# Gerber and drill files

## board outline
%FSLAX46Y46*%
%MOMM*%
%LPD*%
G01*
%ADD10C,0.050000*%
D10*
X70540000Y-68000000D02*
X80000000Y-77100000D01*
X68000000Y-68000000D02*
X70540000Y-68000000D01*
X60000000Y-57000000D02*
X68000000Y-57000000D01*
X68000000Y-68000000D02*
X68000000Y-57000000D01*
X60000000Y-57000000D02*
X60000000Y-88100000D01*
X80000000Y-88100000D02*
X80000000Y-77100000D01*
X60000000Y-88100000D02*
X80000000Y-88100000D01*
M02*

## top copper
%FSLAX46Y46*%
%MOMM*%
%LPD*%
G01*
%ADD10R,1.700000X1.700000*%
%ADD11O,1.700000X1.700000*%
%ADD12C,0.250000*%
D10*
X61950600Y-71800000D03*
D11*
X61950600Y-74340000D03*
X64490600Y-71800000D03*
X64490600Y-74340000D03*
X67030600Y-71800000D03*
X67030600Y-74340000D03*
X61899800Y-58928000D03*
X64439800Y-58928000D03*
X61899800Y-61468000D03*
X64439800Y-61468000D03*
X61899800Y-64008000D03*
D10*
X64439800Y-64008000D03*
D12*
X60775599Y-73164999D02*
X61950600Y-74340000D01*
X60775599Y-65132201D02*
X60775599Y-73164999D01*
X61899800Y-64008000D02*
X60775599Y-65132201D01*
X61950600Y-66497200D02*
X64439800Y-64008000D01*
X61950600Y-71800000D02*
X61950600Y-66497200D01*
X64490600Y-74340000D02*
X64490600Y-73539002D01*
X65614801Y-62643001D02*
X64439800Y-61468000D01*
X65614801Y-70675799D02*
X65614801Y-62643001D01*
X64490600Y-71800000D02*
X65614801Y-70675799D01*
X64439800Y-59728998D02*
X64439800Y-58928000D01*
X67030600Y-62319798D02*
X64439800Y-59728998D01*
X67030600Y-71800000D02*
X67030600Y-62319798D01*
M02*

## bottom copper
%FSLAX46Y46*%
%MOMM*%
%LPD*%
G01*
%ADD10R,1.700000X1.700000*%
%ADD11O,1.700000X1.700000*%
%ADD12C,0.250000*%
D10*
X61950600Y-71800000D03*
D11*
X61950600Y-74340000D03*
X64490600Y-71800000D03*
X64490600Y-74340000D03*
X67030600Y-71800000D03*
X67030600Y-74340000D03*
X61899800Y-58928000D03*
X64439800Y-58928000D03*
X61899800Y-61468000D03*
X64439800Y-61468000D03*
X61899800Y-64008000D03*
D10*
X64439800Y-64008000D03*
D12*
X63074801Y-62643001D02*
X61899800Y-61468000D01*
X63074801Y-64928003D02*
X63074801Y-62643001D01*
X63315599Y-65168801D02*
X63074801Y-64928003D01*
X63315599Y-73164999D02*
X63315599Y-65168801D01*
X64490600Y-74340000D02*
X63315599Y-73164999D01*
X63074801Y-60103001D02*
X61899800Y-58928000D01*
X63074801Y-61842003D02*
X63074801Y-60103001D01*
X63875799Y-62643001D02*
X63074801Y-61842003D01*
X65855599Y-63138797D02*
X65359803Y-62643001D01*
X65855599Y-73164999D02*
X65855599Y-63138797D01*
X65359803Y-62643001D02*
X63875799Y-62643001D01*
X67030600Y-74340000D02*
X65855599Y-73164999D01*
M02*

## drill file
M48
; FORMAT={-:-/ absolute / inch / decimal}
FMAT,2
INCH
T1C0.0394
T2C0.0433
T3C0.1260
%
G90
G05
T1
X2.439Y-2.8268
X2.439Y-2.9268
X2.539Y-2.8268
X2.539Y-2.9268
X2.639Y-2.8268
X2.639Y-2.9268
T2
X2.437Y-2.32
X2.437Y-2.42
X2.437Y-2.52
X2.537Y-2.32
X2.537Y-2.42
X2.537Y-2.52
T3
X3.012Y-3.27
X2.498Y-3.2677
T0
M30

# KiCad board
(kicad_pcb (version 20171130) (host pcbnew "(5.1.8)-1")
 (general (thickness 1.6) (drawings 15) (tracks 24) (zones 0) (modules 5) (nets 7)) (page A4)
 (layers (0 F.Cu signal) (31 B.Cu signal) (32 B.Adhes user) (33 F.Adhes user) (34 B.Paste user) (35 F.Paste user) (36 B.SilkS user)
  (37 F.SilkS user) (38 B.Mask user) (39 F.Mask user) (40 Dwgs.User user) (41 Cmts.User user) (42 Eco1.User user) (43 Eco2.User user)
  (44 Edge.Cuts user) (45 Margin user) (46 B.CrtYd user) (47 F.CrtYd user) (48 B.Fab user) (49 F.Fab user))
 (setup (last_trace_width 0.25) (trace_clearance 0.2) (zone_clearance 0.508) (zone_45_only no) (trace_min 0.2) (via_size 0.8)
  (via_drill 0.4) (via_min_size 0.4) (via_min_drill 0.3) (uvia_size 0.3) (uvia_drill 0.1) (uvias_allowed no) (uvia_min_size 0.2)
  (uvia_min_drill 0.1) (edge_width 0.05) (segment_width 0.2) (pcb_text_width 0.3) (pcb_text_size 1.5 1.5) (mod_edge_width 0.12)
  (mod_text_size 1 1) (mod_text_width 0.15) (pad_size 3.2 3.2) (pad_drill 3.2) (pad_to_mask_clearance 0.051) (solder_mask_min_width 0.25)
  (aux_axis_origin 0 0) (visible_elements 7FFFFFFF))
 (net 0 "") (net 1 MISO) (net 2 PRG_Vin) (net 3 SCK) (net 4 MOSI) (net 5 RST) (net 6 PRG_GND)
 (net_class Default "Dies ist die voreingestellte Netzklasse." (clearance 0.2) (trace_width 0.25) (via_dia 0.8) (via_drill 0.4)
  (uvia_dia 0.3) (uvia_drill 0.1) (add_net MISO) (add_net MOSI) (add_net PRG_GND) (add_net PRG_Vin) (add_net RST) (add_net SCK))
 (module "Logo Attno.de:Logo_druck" (layer F.Cu) (at 69.9262 81.6864)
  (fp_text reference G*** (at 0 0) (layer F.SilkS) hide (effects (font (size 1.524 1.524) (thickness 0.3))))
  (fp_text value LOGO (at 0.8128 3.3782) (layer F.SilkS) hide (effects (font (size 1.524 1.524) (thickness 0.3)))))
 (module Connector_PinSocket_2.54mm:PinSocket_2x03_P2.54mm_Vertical (layer F.Cu) (at 61.9506 71.8 90)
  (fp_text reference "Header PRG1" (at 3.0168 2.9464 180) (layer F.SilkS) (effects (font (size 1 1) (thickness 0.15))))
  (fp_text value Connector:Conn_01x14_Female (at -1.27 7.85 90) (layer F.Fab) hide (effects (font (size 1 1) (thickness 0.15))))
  (pad 1 thru_hole rect (at 0 0 90) (size 1.7 1.7) (drill 1) (layers *.Cu *.Mask) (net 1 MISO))
  (pad 2 thru_hole oval (at -2.54 0 90) (size 1.7 1.7) (drill 1) (layers *.Cu *.Mask) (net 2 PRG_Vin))
  (pad 3 thru_hole oval (at 0 2.54 90) (size 1.7 1.7) (drill 1) (layers *.Cu *.Mask) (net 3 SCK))
  (pad 4 thru_hole oval (at -2.54 2.54 90) (size 1.7 1.7) (drill 1) (layers *.Cu *.Mask) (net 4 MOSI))
  (pad 5 thru_hole oval (at 0 5.08 90) (size 1.7 1.7) (drill 1) (layers *.Cu *.Mask) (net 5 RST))
  (pad 6 thru_hole oval (at -2.54 5.08 90) (size 1.7 1.7) (drill 1) (layers *.Cu *.Mask) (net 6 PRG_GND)))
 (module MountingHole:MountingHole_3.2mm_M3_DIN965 (layer F.Cu) (at 76.5048 83.058)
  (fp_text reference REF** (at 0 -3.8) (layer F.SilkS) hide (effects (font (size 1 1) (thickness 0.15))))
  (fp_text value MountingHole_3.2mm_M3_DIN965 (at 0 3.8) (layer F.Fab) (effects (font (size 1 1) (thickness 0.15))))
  (pad 1 np_thru_hole circle (at 0 0) (size 3.2 3.2) (drill 3.2) (layers *.Cu *.Mask)))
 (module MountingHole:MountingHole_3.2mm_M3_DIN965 (layer F.Cu) (at 63.4492 83)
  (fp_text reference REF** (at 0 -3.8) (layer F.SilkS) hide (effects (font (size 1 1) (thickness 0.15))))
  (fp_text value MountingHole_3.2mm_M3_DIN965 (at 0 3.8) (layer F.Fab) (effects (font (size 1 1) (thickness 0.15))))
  (pad 1 np_thru_hole circle (at 0 0) (size 3.2 3.2) (drill 3.2) (layers *.Cu *.Mask)))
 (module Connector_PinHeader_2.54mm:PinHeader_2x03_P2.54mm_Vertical (layer F.Cu) (at 64.4398 64.008 180)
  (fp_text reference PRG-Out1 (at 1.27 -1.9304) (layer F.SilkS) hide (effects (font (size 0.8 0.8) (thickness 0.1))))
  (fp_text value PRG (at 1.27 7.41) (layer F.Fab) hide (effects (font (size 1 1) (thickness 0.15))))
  (pad 6 thru_hole oval (at 2.54 5.08 180) (size 1.7 1.7) (drill 1.1) (layers *.Cu *.Mask) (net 6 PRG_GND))
  (pad 5 thru_hole oval (at 0 5.08 180) (size 1.7 1.7) (drill 1.1) (layers *.Cu *.Mask) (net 5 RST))
  (pad 4 thru_hole oval (at 2.54 2.54 180) (size 1.7 1.7) (drill 1.1) (layers *.Cu *.Mask) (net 4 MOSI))
  (pad 3 thru_hole oval (at 0 2.54 180) (size 1.7 1.7) (drill 1.1) (layers *.Cu *.Mask) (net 3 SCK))
  (pad 2 thru_hole oval (at 2.54 0 180) (size 1.7 1.7) (drill 1.1) (layers *.Cu *.Mask) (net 2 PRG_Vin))
  (pad 1 thru_hole rect (at 0 0 180) (size 1.7 1.7) (drill 1.1) (layers *.Cu *.Mask) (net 1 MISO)))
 (gr_line (start 70.54 68) (end 80 77.1) (layer Edge.Cuts) (width 0.05))
 (gr_line (start 68 68) (end 70.54 68) (layer Edge.Cuts) (width 0.05))
 (gr_line (start 60 57) (end 68 57) (layer Edge.Cuts) (width 0.05))
 (gr_line (start 68 68) (end 68 57) (layer Edge.Cuts) (width 0.05))
 (gr_line (start 60 57) (end 60 88.1) (layer Edge.Cuts) (width 0.05))
 (gr_line (start 80 88.1) (end 80 77.1) (layer Edge.Cuts) (width 0.05))
 (gr_line (start 60 88.1) (end 80 88.1) (layer Edge.Cuts) (width 0.05))
 (segment (start 60.775599 73.164999) (end 61.9506 74.34) (width 0.25) (layer F.Cu) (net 2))
 (segment (start 60.775599 65.132201) (end 60.775599 73.164999) (width 0.25) (layer F.Cu) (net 2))
 (segment (start 61.8998 64.008) (end 60.775599 65.132201) (width 0.25) (layer F.Cu) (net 2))
 (segment (start 61.9506 66.4972) (end 64.4398 64.008) (width 0.25) (layer F.Cu) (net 1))
 (segment (start 61.9506 71.8) (end 61.9506 66.4972) (width 0.25) (layer F.Cu) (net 1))
 (segment (start 64.4906 74.34) (end 64.4906 73.539002) (width 0.25) (layer F.Cu) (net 4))
 (segment (start 63.074801 62.643001) (end 61.8998 61.468) (width 0.25) (layer B.Cu) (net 4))
 (segment (start 63.074801 64.928003) (end 63.074801 62.643001) (width 0.25) (layer B.Cu) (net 4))
 (segment (start 63.315599 65.168801) (end 63.074801 64.928003) (width 0.25) (layer B.Cu) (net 4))
 (segment (start 63.315599 73.164999) (end 63.315599 65.168801) (width 0.25) (layer B.Cu) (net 4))
 (segment (start 64.4906 74.34) (end 63.315599 73.164999) (width 0.25) (layer B.Cu) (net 4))
 (segment (start 65.614801 62.643001) (end 64.4398 61.468) (width 0.25) (layer F.Cu) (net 3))
 (segment (start 65.614801 70.675799) (end 65.614801 62.643001) (width 0.25) (layer F.Cu) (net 3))
 (segment (start 64.4906 71.8) (end 65.614801 70.675799) (width 0.25) (layer F.Cu) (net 3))
 (segment (start 64.4398 59.728998) (end 64.4398 58.928) (width 0.25) (layer F.Cu) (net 5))
 (segment (start 67.0306 62.319798) (end 64.4398 59.728998) (width 0.25) (layer F.Cu) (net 5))
 (segment (start 67.0306 71.8) (end 67.0306 62.319798) (width 0.25) (layer F.Cu) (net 5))
 (segment (start 63.074801 60.103001) (end 61.8998 58.928) (width 0.25) (layer B.Cu) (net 6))
 (segment (start 63.074801 61.842003) (end 63.074801 60.103001) (width 0.25) (layer B.Cu) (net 6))
 (segment (start 63.875799 62.643001) (end 63.074801 61.842003) (width 0.25) (layer B.Cu) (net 6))
 (segment (start 65.855599 63.138797) (end 65.359803 62.643001) (width 0.25) (layer B.Cu) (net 6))
 (segment (start 65.855599 73.164999) (end 65.855599 63.138797) (width 0.25) (layer B.Cu) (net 6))
 (segment (start 65.359803 62.643001) (end 63.875799 62.643001) (width 0.25) (layer B.Cu) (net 6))
 (segment (start 67.0306 74.34) (end 65.855599 73.164999) (width 0.25) (layer B.Cu) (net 6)))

